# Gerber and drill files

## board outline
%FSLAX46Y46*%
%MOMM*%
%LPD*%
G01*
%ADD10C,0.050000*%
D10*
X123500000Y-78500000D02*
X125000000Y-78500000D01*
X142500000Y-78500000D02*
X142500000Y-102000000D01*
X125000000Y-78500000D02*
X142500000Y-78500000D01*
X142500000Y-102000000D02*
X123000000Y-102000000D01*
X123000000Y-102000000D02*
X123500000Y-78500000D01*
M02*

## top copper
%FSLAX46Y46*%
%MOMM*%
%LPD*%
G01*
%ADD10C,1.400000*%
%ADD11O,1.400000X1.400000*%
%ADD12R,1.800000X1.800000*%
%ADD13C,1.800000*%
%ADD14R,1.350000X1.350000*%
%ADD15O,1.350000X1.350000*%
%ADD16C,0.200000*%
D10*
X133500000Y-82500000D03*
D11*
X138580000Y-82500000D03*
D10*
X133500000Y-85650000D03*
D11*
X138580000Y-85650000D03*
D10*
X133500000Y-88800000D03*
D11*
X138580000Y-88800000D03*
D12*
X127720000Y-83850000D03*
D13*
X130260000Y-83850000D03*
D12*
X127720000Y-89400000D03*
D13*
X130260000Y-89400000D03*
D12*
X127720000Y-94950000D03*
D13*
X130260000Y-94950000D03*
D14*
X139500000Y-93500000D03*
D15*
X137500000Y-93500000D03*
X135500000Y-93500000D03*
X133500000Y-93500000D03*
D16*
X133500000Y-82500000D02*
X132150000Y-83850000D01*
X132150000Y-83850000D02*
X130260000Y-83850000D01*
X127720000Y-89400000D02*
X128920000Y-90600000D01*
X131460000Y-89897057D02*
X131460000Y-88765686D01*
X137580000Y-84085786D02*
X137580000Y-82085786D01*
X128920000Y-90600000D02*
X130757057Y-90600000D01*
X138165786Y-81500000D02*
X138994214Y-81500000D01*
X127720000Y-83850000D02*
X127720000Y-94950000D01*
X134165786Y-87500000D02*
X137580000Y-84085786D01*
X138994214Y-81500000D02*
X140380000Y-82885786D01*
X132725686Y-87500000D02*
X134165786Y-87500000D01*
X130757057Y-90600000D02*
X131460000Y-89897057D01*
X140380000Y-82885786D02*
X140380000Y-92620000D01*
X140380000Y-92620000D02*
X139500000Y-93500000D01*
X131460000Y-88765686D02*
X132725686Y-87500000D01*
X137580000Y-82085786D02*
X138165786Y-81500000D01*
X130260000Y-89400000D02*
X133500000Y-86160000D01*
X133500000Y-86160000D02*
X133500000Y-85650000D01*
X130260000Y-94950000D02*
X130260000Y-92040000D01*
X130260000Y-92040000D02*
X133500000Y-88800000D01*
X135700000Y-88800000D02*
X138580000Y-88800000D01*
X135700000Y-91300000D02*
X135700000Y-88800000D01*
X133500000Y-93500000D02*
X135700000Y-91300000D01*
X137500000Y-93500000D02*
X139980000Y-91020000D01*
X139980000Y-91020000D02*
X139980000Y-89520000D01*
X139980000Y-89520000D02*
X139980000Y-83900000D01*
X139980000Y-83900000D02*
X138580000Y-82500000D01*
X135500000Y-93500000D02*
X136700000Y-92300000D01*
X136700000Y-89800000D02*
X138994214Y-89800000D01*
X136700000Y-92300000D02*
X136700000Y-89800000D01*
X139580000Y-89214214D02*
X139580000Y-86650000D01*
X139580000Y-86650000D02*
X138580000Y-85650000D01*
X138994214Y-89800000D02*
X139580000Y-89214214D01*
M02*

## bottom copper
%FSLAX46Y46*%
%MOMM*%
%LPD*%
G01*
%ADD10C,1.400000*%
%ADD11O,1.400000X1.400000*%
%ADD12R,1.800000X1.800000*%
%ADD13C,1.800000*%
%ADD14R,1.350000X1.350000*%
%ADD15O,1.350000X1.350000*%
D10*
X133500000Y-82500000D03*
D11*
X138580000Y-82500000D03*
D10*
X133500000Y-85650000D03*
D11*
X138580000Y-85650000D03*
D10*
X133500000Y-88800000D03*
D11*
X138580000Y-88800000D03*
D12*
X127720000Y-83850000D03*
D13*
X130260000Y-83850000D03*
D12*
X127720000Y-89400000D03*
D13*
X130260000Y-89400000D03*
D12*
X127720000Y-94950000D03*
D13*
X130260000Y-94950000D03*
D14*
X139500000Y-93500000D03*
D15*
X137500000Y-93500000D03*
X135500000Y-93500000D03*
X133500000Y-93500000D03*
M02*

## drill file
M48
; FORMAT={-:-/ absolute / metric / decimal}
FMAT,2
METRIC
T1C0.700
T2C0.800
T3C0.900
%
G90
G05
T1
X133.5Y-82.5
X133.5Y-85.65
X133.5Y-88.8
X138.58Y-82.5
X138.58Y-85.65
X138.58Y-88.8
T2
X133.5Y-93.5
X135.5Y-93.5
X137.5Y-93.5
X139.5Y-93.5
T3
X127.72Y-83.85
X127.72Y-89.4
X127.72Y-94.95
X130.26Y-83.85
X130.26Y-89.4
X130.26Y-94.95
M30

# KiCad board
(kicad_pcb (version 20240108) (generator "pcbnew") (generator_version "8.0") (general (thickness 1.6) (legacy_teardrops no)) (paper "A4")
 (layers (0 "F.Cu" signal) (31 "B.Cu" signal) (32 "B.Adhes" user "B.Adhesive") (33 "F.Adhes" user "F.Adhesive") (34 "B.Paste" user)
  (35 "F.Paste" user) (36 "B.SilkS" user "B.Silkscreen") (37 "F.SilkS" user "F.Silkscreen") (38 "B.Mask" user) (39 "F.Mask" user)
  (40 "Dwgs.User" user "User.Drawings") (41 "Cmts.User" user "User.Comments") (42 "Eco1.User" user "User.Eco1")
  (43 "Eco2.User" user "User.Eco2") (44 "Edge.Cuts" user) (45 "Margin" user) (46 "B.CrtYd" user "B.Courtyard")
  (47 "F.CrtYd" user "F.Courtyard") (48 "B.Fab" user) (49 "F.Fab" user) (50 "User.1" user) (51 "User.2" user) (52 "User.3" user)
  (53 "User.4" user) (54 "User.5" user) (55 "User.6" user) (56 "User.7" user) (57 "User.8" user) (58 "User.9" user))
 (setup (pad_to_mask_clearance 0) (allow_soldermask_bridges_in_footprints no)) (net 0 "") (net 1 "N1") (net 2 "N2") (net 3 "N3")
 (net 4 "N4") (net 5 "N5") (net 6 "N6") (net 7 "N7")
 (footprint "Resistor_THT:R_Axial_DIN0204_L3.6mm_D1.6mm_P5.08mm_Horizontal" (layer "F.Cu") (at 133.5 82.5)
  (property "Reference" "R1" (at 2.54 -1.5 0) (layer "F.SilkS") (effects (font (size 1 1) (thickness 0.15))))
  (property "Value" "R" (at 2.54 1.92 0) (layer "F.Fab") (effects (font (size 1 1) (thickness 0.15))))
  (pad "1" thru_hole circle (at 0 0) (size 1.4 1.4) (drill 0.7) (layers "*.Cu" "*.Mask") (remove_unused_layers no) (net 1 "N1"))
  (pad "2" thru_hole oval (at 5.08 0) (size 1.4 1.4) (drill 0.7) (layers "*.Cu" "*.Mask") (remove_unused_layers no) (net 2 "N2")))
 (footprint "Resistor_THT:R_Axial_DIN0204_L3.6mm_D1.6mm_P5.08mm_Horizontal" (layer "F.Cu") (at 133.5 85.65)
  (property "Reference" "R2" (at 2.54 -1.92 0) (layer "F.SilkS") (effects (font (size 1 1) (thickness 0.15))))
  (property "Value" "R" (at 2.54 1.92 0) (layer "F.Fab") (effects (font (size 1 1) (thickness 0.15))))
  (pad "1" thru_hole circle (at 0 0) (size 1.4 1.4) (drill 0.7) (layers "*.Cu" "*.Mask") (remove_unused_layers no) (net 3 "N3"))
  (pad "2" thru_hole oval (at 5.08 0) (size 1.4 1.4) (drill 0.7) (layers "*.Cu" "*.Mask") (remove_unused_layers no) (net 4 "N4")))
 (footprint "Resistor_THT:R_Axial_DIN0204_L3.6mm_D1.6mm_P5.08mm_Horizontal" (layer "F.Cu") (at 133.5 88.8)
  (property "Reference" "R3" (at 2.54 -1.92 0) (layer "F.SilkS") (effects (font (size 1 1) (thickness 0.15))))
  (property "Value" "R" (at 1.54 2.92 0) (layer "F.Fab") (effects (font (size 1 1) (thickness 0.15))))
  (pad "1" thru_hole circle (at 0 0) (size 1.4 1.4) (drill 0.7) (layers "*.Cu" "*.Mask") (remove_unused_layers no) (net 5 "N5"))
  (pad "2" thru_hole oval (at 5.08 0) (size 1.4 1.4) (drill 0.7) (layers "*.Cu" "*.Mask") (remove_unused_layers no) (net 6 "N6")))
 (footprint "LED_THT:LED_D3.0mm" (layer "F.Cu") (at 127.72 83.85)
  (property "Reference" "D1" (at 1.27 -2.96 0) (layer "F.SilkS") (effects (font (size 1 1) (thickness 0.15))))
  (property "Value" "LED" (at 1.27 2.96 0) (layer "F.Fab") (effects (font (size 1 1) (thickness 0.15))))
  (pad "1" thru_hole rect (at 0 0) (size 1.8 1.8) (drill 0.9) (layers "*.Cu" "*.Mask") (remove_unused_layers no) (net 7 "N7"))
  (pad "2" thru_hole circle (at 2.54 0) (size 1.8 1.8) (drill 0.9) (layers "*.Cu" "*.Mask") (remove_unused_layers no) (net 1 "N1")))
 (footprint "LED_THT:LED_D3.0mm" (layer "F.Cu") (at 127.72 89.4)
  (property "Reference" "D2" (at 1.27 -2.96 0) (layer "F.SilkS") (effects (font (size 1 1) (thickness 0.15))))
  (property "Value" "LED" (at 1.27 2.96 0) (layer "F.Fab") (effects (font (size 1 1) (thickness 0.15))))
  (pad "1" thru_hole rect (at 0 0) (size 1.8 1.8) (drill 0.9) (layers "*.Cu" "*.Mask") (remove_unused_layers no) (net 7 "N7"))
  (pad "2" thru_hole circle (at 2.54 0) (size 1.8 1.8) (drill 0.9) (layers "*.Cu" "*.Mask") (remove_unused_layers no) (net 3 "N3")))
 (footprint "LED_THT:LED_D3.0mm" (layer "F.Cu") (at 127.72 94.95)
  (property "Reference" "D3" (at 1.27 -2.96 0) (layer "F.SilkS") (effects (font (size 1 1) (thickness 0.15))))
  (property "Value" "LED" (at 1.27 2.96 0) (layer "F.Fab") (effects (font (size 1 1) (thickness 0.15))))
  (pad "1" thru_hole rect (at 0 0) (size 1.8 1.8) (drill 0.9) (layers "*.Cu" "*.Mask") (remove_unused_layers no) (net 7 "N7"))
  (pad "2" thru_hole circle (at 2.54 0) (size 1.8 1.8) (drill 0.9) (layers "*.Cu" "*.Mask") (remove_unused_layers no) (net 5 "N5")))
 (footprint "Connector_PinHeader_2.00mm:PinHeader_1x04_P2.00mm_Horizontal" (layer "F.Cu") (at 139.5 93.5 -90)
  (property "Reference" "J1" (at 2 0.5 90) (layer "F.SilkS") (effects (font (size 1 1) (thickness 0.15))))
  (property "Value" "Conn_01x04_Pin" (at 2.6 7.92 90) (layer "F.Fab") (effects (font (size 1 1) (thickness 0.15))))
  (pad "1" thru_hole rect (at 0 0 270) (size 1.35 1.35) (drill 0.8) (layers "*.Cu" "*.Mask") (remove_unused_layers no) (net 7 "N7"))
  (pad "2" thru_hole oval (at 0 2 270) (size 1.35 1.35) (drill 0.8) (layers "*.Cu" "*.Mask") (remove_unused_layers no) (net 2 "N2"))
  (pad "3" thru_hole oval (at 0 4 270) (size 1.35 1.35) (drill 0.8) (layers "*.Cu" "*.Mask") (remove_unused_layers no) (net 4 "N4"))
  (pad "4" thru_hole oval (at 0 6 270) (size 1.35 1.35) (drill 0.8) (layers "*.Cu" "*.Mask") (remove_unused_layers no) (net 6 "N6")))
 (gr_line (start 123.5 78.5) (end 125 78.5) (stroke (width 0.05) (type default)) (layer "Edge.Cuts"))
 (gr_line (start 142.5 78.5) (end 142.5 102) (stroke (width 0.05) (type default)) (layer "Edge.Cuts"))
 (gr_line (start 125 78.5) (end 142.5 78.5) (stroke (width 0.05) (type default)) (layer "Edge.Cuts"))
 (gr_line (start 142.5 102) (end 123 102) (stroke (width 0.05) (type default)) (layer "Edge.Cuts"))
 (gr_line (start 123 102) (end 123.5 78.5) (stroke (width 0.05) (type default)) (layer "Edge.Cuts"))
 (segment (start 133.5 82.5) (end 132.15 83.85) (width 0.2) (layer "F.Cu") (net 1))
 (segment (start 132.15 83.85) (end 130.26 83.85) (width 0.2) (layer "F.Cu") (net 1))
 (segment (start 127.72 89.4) (end 128.92 90.6) (width 0.2) (layer "F.Cu") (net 7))
 (segment (start 131.46 89.897057) (end 131.46 88.765686) (width 0.2) (layer "F.Cu") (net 7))
 (segment (start 137.58 84.085786) (end 137.58 82.085786) (width 0.2) (layer "F.Cu") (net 7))
 (segment (start 128.92 90.6) (end 130.757057 90.6) (width 0.2) (layer "F.Cu") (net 7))
 (segment (start 138.165786 81.5) (end 138.994214 81.5) (width 0.2) (layer "F.Cu") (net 7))
 (segment (start 127.72 83.85) (end 127.72 94.95) (width 0.2) (layer "F.Cu") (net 7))
 (segment (start 134.165786 87.5) (end 137.58 84.085786) (width 0.2) (layer "F.Cu") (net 7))
 (segment (start 138.994214 81.5) (end 140.38 82.885786) (width 0.2) (layer "F.Cu") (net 7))
 (segment (start 132.725686 87.5) (end 134.165786 87.5) (width 0.2) (layer "F.Cu") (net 7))
 (segment (start 130.757057 90.6) (end 131.46 89.897057) (width 0.2) (layer "F.Cu") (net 7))
 (segment (start 140.38 82.885786) (end 140.38 92.62) (width 0.2) (layer "F.Cu") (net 7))
 (segment (start 140.38 92.62) (end 139.5 93.5) (width 0.2) (layer "F.Cu") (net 7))
 (segment (start 131.46 88.765686) (end 132.725686 87.5) (width 0.2) (layer "F.Cu") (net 7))
 (segment (start 137.58 82.085786) (end 138.165786 81.5) (width 0.2) (layer "F.Cu") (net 7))
 (segment (start 130.26 89.4) (end 133.5 86.16) (width 0.2) (layer "F.Cu") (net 3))
 (segment (start 133.5 86.16) (end 133.5 85.65) (width 0.2) (layer "F.Cu") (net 3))
 (segment (start 130.26 94.95) (end 130.26 92.04) (width 0.2) (layer "F.Cu") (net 5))
 (segment (start 130.26 92.04) (end 133.5 88.8) (width 0.2) (layer "F.Cu") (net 5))
 (segment (start 135.7 88.8) (end 138.58 88.8) (width 0.2) (layer "F.Cu") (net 6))
 (segment (start 135.7 91.3) (end 135.7 88.8) (width 0.2) (layer "F.Cu") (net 6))
 (segment (start 133.5 93.5) (end 135.7 91.3) (width 0.2) (layer "F.Cu") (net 6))
 (segment (start 137.5 93.5) (end 139.98 91.02) (width 0.2) (layer "F.Cu") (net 2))
 (segment (start 139.98 91.02) (end 139.98 89.52) (width 0.2) (layer "F.Cu") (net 2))
 (segment (start 139.98 89.52) (end 139.98 83.9) (width 0.2) (layer "F.Cu") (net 2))
 (segment (start 139.98 83.9) (end 138.58 82.5) (width 0.2) (layer "F.Cu") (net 2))
 (segment (start 135.5 93.5) (end 136.7 92.3) (width 0.2) (layer "F.Cu") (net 4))
 (segment (start 136.7 89.8) (end 138.994214 89.8) (width 0.2) (layer "F.Cu") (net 4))
 (segment (start 136.7 92.3) (end 136.7 89.8) (width 0.2) (layer "F.Cu") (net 4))
 (segment (start 139.58 89.214214) (end 139.58 86.65) (width 0.2) (layer "F.Cu") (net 4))
 (segment (start 139.58 86.65) (end 138.58 85.65) (width 0.2) (layer "F.Cu") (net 4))
 (segment (start 138.994214 89.8) (end 139.58 89.214214) (width 0.2) (layer "F.Cu") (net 4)))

